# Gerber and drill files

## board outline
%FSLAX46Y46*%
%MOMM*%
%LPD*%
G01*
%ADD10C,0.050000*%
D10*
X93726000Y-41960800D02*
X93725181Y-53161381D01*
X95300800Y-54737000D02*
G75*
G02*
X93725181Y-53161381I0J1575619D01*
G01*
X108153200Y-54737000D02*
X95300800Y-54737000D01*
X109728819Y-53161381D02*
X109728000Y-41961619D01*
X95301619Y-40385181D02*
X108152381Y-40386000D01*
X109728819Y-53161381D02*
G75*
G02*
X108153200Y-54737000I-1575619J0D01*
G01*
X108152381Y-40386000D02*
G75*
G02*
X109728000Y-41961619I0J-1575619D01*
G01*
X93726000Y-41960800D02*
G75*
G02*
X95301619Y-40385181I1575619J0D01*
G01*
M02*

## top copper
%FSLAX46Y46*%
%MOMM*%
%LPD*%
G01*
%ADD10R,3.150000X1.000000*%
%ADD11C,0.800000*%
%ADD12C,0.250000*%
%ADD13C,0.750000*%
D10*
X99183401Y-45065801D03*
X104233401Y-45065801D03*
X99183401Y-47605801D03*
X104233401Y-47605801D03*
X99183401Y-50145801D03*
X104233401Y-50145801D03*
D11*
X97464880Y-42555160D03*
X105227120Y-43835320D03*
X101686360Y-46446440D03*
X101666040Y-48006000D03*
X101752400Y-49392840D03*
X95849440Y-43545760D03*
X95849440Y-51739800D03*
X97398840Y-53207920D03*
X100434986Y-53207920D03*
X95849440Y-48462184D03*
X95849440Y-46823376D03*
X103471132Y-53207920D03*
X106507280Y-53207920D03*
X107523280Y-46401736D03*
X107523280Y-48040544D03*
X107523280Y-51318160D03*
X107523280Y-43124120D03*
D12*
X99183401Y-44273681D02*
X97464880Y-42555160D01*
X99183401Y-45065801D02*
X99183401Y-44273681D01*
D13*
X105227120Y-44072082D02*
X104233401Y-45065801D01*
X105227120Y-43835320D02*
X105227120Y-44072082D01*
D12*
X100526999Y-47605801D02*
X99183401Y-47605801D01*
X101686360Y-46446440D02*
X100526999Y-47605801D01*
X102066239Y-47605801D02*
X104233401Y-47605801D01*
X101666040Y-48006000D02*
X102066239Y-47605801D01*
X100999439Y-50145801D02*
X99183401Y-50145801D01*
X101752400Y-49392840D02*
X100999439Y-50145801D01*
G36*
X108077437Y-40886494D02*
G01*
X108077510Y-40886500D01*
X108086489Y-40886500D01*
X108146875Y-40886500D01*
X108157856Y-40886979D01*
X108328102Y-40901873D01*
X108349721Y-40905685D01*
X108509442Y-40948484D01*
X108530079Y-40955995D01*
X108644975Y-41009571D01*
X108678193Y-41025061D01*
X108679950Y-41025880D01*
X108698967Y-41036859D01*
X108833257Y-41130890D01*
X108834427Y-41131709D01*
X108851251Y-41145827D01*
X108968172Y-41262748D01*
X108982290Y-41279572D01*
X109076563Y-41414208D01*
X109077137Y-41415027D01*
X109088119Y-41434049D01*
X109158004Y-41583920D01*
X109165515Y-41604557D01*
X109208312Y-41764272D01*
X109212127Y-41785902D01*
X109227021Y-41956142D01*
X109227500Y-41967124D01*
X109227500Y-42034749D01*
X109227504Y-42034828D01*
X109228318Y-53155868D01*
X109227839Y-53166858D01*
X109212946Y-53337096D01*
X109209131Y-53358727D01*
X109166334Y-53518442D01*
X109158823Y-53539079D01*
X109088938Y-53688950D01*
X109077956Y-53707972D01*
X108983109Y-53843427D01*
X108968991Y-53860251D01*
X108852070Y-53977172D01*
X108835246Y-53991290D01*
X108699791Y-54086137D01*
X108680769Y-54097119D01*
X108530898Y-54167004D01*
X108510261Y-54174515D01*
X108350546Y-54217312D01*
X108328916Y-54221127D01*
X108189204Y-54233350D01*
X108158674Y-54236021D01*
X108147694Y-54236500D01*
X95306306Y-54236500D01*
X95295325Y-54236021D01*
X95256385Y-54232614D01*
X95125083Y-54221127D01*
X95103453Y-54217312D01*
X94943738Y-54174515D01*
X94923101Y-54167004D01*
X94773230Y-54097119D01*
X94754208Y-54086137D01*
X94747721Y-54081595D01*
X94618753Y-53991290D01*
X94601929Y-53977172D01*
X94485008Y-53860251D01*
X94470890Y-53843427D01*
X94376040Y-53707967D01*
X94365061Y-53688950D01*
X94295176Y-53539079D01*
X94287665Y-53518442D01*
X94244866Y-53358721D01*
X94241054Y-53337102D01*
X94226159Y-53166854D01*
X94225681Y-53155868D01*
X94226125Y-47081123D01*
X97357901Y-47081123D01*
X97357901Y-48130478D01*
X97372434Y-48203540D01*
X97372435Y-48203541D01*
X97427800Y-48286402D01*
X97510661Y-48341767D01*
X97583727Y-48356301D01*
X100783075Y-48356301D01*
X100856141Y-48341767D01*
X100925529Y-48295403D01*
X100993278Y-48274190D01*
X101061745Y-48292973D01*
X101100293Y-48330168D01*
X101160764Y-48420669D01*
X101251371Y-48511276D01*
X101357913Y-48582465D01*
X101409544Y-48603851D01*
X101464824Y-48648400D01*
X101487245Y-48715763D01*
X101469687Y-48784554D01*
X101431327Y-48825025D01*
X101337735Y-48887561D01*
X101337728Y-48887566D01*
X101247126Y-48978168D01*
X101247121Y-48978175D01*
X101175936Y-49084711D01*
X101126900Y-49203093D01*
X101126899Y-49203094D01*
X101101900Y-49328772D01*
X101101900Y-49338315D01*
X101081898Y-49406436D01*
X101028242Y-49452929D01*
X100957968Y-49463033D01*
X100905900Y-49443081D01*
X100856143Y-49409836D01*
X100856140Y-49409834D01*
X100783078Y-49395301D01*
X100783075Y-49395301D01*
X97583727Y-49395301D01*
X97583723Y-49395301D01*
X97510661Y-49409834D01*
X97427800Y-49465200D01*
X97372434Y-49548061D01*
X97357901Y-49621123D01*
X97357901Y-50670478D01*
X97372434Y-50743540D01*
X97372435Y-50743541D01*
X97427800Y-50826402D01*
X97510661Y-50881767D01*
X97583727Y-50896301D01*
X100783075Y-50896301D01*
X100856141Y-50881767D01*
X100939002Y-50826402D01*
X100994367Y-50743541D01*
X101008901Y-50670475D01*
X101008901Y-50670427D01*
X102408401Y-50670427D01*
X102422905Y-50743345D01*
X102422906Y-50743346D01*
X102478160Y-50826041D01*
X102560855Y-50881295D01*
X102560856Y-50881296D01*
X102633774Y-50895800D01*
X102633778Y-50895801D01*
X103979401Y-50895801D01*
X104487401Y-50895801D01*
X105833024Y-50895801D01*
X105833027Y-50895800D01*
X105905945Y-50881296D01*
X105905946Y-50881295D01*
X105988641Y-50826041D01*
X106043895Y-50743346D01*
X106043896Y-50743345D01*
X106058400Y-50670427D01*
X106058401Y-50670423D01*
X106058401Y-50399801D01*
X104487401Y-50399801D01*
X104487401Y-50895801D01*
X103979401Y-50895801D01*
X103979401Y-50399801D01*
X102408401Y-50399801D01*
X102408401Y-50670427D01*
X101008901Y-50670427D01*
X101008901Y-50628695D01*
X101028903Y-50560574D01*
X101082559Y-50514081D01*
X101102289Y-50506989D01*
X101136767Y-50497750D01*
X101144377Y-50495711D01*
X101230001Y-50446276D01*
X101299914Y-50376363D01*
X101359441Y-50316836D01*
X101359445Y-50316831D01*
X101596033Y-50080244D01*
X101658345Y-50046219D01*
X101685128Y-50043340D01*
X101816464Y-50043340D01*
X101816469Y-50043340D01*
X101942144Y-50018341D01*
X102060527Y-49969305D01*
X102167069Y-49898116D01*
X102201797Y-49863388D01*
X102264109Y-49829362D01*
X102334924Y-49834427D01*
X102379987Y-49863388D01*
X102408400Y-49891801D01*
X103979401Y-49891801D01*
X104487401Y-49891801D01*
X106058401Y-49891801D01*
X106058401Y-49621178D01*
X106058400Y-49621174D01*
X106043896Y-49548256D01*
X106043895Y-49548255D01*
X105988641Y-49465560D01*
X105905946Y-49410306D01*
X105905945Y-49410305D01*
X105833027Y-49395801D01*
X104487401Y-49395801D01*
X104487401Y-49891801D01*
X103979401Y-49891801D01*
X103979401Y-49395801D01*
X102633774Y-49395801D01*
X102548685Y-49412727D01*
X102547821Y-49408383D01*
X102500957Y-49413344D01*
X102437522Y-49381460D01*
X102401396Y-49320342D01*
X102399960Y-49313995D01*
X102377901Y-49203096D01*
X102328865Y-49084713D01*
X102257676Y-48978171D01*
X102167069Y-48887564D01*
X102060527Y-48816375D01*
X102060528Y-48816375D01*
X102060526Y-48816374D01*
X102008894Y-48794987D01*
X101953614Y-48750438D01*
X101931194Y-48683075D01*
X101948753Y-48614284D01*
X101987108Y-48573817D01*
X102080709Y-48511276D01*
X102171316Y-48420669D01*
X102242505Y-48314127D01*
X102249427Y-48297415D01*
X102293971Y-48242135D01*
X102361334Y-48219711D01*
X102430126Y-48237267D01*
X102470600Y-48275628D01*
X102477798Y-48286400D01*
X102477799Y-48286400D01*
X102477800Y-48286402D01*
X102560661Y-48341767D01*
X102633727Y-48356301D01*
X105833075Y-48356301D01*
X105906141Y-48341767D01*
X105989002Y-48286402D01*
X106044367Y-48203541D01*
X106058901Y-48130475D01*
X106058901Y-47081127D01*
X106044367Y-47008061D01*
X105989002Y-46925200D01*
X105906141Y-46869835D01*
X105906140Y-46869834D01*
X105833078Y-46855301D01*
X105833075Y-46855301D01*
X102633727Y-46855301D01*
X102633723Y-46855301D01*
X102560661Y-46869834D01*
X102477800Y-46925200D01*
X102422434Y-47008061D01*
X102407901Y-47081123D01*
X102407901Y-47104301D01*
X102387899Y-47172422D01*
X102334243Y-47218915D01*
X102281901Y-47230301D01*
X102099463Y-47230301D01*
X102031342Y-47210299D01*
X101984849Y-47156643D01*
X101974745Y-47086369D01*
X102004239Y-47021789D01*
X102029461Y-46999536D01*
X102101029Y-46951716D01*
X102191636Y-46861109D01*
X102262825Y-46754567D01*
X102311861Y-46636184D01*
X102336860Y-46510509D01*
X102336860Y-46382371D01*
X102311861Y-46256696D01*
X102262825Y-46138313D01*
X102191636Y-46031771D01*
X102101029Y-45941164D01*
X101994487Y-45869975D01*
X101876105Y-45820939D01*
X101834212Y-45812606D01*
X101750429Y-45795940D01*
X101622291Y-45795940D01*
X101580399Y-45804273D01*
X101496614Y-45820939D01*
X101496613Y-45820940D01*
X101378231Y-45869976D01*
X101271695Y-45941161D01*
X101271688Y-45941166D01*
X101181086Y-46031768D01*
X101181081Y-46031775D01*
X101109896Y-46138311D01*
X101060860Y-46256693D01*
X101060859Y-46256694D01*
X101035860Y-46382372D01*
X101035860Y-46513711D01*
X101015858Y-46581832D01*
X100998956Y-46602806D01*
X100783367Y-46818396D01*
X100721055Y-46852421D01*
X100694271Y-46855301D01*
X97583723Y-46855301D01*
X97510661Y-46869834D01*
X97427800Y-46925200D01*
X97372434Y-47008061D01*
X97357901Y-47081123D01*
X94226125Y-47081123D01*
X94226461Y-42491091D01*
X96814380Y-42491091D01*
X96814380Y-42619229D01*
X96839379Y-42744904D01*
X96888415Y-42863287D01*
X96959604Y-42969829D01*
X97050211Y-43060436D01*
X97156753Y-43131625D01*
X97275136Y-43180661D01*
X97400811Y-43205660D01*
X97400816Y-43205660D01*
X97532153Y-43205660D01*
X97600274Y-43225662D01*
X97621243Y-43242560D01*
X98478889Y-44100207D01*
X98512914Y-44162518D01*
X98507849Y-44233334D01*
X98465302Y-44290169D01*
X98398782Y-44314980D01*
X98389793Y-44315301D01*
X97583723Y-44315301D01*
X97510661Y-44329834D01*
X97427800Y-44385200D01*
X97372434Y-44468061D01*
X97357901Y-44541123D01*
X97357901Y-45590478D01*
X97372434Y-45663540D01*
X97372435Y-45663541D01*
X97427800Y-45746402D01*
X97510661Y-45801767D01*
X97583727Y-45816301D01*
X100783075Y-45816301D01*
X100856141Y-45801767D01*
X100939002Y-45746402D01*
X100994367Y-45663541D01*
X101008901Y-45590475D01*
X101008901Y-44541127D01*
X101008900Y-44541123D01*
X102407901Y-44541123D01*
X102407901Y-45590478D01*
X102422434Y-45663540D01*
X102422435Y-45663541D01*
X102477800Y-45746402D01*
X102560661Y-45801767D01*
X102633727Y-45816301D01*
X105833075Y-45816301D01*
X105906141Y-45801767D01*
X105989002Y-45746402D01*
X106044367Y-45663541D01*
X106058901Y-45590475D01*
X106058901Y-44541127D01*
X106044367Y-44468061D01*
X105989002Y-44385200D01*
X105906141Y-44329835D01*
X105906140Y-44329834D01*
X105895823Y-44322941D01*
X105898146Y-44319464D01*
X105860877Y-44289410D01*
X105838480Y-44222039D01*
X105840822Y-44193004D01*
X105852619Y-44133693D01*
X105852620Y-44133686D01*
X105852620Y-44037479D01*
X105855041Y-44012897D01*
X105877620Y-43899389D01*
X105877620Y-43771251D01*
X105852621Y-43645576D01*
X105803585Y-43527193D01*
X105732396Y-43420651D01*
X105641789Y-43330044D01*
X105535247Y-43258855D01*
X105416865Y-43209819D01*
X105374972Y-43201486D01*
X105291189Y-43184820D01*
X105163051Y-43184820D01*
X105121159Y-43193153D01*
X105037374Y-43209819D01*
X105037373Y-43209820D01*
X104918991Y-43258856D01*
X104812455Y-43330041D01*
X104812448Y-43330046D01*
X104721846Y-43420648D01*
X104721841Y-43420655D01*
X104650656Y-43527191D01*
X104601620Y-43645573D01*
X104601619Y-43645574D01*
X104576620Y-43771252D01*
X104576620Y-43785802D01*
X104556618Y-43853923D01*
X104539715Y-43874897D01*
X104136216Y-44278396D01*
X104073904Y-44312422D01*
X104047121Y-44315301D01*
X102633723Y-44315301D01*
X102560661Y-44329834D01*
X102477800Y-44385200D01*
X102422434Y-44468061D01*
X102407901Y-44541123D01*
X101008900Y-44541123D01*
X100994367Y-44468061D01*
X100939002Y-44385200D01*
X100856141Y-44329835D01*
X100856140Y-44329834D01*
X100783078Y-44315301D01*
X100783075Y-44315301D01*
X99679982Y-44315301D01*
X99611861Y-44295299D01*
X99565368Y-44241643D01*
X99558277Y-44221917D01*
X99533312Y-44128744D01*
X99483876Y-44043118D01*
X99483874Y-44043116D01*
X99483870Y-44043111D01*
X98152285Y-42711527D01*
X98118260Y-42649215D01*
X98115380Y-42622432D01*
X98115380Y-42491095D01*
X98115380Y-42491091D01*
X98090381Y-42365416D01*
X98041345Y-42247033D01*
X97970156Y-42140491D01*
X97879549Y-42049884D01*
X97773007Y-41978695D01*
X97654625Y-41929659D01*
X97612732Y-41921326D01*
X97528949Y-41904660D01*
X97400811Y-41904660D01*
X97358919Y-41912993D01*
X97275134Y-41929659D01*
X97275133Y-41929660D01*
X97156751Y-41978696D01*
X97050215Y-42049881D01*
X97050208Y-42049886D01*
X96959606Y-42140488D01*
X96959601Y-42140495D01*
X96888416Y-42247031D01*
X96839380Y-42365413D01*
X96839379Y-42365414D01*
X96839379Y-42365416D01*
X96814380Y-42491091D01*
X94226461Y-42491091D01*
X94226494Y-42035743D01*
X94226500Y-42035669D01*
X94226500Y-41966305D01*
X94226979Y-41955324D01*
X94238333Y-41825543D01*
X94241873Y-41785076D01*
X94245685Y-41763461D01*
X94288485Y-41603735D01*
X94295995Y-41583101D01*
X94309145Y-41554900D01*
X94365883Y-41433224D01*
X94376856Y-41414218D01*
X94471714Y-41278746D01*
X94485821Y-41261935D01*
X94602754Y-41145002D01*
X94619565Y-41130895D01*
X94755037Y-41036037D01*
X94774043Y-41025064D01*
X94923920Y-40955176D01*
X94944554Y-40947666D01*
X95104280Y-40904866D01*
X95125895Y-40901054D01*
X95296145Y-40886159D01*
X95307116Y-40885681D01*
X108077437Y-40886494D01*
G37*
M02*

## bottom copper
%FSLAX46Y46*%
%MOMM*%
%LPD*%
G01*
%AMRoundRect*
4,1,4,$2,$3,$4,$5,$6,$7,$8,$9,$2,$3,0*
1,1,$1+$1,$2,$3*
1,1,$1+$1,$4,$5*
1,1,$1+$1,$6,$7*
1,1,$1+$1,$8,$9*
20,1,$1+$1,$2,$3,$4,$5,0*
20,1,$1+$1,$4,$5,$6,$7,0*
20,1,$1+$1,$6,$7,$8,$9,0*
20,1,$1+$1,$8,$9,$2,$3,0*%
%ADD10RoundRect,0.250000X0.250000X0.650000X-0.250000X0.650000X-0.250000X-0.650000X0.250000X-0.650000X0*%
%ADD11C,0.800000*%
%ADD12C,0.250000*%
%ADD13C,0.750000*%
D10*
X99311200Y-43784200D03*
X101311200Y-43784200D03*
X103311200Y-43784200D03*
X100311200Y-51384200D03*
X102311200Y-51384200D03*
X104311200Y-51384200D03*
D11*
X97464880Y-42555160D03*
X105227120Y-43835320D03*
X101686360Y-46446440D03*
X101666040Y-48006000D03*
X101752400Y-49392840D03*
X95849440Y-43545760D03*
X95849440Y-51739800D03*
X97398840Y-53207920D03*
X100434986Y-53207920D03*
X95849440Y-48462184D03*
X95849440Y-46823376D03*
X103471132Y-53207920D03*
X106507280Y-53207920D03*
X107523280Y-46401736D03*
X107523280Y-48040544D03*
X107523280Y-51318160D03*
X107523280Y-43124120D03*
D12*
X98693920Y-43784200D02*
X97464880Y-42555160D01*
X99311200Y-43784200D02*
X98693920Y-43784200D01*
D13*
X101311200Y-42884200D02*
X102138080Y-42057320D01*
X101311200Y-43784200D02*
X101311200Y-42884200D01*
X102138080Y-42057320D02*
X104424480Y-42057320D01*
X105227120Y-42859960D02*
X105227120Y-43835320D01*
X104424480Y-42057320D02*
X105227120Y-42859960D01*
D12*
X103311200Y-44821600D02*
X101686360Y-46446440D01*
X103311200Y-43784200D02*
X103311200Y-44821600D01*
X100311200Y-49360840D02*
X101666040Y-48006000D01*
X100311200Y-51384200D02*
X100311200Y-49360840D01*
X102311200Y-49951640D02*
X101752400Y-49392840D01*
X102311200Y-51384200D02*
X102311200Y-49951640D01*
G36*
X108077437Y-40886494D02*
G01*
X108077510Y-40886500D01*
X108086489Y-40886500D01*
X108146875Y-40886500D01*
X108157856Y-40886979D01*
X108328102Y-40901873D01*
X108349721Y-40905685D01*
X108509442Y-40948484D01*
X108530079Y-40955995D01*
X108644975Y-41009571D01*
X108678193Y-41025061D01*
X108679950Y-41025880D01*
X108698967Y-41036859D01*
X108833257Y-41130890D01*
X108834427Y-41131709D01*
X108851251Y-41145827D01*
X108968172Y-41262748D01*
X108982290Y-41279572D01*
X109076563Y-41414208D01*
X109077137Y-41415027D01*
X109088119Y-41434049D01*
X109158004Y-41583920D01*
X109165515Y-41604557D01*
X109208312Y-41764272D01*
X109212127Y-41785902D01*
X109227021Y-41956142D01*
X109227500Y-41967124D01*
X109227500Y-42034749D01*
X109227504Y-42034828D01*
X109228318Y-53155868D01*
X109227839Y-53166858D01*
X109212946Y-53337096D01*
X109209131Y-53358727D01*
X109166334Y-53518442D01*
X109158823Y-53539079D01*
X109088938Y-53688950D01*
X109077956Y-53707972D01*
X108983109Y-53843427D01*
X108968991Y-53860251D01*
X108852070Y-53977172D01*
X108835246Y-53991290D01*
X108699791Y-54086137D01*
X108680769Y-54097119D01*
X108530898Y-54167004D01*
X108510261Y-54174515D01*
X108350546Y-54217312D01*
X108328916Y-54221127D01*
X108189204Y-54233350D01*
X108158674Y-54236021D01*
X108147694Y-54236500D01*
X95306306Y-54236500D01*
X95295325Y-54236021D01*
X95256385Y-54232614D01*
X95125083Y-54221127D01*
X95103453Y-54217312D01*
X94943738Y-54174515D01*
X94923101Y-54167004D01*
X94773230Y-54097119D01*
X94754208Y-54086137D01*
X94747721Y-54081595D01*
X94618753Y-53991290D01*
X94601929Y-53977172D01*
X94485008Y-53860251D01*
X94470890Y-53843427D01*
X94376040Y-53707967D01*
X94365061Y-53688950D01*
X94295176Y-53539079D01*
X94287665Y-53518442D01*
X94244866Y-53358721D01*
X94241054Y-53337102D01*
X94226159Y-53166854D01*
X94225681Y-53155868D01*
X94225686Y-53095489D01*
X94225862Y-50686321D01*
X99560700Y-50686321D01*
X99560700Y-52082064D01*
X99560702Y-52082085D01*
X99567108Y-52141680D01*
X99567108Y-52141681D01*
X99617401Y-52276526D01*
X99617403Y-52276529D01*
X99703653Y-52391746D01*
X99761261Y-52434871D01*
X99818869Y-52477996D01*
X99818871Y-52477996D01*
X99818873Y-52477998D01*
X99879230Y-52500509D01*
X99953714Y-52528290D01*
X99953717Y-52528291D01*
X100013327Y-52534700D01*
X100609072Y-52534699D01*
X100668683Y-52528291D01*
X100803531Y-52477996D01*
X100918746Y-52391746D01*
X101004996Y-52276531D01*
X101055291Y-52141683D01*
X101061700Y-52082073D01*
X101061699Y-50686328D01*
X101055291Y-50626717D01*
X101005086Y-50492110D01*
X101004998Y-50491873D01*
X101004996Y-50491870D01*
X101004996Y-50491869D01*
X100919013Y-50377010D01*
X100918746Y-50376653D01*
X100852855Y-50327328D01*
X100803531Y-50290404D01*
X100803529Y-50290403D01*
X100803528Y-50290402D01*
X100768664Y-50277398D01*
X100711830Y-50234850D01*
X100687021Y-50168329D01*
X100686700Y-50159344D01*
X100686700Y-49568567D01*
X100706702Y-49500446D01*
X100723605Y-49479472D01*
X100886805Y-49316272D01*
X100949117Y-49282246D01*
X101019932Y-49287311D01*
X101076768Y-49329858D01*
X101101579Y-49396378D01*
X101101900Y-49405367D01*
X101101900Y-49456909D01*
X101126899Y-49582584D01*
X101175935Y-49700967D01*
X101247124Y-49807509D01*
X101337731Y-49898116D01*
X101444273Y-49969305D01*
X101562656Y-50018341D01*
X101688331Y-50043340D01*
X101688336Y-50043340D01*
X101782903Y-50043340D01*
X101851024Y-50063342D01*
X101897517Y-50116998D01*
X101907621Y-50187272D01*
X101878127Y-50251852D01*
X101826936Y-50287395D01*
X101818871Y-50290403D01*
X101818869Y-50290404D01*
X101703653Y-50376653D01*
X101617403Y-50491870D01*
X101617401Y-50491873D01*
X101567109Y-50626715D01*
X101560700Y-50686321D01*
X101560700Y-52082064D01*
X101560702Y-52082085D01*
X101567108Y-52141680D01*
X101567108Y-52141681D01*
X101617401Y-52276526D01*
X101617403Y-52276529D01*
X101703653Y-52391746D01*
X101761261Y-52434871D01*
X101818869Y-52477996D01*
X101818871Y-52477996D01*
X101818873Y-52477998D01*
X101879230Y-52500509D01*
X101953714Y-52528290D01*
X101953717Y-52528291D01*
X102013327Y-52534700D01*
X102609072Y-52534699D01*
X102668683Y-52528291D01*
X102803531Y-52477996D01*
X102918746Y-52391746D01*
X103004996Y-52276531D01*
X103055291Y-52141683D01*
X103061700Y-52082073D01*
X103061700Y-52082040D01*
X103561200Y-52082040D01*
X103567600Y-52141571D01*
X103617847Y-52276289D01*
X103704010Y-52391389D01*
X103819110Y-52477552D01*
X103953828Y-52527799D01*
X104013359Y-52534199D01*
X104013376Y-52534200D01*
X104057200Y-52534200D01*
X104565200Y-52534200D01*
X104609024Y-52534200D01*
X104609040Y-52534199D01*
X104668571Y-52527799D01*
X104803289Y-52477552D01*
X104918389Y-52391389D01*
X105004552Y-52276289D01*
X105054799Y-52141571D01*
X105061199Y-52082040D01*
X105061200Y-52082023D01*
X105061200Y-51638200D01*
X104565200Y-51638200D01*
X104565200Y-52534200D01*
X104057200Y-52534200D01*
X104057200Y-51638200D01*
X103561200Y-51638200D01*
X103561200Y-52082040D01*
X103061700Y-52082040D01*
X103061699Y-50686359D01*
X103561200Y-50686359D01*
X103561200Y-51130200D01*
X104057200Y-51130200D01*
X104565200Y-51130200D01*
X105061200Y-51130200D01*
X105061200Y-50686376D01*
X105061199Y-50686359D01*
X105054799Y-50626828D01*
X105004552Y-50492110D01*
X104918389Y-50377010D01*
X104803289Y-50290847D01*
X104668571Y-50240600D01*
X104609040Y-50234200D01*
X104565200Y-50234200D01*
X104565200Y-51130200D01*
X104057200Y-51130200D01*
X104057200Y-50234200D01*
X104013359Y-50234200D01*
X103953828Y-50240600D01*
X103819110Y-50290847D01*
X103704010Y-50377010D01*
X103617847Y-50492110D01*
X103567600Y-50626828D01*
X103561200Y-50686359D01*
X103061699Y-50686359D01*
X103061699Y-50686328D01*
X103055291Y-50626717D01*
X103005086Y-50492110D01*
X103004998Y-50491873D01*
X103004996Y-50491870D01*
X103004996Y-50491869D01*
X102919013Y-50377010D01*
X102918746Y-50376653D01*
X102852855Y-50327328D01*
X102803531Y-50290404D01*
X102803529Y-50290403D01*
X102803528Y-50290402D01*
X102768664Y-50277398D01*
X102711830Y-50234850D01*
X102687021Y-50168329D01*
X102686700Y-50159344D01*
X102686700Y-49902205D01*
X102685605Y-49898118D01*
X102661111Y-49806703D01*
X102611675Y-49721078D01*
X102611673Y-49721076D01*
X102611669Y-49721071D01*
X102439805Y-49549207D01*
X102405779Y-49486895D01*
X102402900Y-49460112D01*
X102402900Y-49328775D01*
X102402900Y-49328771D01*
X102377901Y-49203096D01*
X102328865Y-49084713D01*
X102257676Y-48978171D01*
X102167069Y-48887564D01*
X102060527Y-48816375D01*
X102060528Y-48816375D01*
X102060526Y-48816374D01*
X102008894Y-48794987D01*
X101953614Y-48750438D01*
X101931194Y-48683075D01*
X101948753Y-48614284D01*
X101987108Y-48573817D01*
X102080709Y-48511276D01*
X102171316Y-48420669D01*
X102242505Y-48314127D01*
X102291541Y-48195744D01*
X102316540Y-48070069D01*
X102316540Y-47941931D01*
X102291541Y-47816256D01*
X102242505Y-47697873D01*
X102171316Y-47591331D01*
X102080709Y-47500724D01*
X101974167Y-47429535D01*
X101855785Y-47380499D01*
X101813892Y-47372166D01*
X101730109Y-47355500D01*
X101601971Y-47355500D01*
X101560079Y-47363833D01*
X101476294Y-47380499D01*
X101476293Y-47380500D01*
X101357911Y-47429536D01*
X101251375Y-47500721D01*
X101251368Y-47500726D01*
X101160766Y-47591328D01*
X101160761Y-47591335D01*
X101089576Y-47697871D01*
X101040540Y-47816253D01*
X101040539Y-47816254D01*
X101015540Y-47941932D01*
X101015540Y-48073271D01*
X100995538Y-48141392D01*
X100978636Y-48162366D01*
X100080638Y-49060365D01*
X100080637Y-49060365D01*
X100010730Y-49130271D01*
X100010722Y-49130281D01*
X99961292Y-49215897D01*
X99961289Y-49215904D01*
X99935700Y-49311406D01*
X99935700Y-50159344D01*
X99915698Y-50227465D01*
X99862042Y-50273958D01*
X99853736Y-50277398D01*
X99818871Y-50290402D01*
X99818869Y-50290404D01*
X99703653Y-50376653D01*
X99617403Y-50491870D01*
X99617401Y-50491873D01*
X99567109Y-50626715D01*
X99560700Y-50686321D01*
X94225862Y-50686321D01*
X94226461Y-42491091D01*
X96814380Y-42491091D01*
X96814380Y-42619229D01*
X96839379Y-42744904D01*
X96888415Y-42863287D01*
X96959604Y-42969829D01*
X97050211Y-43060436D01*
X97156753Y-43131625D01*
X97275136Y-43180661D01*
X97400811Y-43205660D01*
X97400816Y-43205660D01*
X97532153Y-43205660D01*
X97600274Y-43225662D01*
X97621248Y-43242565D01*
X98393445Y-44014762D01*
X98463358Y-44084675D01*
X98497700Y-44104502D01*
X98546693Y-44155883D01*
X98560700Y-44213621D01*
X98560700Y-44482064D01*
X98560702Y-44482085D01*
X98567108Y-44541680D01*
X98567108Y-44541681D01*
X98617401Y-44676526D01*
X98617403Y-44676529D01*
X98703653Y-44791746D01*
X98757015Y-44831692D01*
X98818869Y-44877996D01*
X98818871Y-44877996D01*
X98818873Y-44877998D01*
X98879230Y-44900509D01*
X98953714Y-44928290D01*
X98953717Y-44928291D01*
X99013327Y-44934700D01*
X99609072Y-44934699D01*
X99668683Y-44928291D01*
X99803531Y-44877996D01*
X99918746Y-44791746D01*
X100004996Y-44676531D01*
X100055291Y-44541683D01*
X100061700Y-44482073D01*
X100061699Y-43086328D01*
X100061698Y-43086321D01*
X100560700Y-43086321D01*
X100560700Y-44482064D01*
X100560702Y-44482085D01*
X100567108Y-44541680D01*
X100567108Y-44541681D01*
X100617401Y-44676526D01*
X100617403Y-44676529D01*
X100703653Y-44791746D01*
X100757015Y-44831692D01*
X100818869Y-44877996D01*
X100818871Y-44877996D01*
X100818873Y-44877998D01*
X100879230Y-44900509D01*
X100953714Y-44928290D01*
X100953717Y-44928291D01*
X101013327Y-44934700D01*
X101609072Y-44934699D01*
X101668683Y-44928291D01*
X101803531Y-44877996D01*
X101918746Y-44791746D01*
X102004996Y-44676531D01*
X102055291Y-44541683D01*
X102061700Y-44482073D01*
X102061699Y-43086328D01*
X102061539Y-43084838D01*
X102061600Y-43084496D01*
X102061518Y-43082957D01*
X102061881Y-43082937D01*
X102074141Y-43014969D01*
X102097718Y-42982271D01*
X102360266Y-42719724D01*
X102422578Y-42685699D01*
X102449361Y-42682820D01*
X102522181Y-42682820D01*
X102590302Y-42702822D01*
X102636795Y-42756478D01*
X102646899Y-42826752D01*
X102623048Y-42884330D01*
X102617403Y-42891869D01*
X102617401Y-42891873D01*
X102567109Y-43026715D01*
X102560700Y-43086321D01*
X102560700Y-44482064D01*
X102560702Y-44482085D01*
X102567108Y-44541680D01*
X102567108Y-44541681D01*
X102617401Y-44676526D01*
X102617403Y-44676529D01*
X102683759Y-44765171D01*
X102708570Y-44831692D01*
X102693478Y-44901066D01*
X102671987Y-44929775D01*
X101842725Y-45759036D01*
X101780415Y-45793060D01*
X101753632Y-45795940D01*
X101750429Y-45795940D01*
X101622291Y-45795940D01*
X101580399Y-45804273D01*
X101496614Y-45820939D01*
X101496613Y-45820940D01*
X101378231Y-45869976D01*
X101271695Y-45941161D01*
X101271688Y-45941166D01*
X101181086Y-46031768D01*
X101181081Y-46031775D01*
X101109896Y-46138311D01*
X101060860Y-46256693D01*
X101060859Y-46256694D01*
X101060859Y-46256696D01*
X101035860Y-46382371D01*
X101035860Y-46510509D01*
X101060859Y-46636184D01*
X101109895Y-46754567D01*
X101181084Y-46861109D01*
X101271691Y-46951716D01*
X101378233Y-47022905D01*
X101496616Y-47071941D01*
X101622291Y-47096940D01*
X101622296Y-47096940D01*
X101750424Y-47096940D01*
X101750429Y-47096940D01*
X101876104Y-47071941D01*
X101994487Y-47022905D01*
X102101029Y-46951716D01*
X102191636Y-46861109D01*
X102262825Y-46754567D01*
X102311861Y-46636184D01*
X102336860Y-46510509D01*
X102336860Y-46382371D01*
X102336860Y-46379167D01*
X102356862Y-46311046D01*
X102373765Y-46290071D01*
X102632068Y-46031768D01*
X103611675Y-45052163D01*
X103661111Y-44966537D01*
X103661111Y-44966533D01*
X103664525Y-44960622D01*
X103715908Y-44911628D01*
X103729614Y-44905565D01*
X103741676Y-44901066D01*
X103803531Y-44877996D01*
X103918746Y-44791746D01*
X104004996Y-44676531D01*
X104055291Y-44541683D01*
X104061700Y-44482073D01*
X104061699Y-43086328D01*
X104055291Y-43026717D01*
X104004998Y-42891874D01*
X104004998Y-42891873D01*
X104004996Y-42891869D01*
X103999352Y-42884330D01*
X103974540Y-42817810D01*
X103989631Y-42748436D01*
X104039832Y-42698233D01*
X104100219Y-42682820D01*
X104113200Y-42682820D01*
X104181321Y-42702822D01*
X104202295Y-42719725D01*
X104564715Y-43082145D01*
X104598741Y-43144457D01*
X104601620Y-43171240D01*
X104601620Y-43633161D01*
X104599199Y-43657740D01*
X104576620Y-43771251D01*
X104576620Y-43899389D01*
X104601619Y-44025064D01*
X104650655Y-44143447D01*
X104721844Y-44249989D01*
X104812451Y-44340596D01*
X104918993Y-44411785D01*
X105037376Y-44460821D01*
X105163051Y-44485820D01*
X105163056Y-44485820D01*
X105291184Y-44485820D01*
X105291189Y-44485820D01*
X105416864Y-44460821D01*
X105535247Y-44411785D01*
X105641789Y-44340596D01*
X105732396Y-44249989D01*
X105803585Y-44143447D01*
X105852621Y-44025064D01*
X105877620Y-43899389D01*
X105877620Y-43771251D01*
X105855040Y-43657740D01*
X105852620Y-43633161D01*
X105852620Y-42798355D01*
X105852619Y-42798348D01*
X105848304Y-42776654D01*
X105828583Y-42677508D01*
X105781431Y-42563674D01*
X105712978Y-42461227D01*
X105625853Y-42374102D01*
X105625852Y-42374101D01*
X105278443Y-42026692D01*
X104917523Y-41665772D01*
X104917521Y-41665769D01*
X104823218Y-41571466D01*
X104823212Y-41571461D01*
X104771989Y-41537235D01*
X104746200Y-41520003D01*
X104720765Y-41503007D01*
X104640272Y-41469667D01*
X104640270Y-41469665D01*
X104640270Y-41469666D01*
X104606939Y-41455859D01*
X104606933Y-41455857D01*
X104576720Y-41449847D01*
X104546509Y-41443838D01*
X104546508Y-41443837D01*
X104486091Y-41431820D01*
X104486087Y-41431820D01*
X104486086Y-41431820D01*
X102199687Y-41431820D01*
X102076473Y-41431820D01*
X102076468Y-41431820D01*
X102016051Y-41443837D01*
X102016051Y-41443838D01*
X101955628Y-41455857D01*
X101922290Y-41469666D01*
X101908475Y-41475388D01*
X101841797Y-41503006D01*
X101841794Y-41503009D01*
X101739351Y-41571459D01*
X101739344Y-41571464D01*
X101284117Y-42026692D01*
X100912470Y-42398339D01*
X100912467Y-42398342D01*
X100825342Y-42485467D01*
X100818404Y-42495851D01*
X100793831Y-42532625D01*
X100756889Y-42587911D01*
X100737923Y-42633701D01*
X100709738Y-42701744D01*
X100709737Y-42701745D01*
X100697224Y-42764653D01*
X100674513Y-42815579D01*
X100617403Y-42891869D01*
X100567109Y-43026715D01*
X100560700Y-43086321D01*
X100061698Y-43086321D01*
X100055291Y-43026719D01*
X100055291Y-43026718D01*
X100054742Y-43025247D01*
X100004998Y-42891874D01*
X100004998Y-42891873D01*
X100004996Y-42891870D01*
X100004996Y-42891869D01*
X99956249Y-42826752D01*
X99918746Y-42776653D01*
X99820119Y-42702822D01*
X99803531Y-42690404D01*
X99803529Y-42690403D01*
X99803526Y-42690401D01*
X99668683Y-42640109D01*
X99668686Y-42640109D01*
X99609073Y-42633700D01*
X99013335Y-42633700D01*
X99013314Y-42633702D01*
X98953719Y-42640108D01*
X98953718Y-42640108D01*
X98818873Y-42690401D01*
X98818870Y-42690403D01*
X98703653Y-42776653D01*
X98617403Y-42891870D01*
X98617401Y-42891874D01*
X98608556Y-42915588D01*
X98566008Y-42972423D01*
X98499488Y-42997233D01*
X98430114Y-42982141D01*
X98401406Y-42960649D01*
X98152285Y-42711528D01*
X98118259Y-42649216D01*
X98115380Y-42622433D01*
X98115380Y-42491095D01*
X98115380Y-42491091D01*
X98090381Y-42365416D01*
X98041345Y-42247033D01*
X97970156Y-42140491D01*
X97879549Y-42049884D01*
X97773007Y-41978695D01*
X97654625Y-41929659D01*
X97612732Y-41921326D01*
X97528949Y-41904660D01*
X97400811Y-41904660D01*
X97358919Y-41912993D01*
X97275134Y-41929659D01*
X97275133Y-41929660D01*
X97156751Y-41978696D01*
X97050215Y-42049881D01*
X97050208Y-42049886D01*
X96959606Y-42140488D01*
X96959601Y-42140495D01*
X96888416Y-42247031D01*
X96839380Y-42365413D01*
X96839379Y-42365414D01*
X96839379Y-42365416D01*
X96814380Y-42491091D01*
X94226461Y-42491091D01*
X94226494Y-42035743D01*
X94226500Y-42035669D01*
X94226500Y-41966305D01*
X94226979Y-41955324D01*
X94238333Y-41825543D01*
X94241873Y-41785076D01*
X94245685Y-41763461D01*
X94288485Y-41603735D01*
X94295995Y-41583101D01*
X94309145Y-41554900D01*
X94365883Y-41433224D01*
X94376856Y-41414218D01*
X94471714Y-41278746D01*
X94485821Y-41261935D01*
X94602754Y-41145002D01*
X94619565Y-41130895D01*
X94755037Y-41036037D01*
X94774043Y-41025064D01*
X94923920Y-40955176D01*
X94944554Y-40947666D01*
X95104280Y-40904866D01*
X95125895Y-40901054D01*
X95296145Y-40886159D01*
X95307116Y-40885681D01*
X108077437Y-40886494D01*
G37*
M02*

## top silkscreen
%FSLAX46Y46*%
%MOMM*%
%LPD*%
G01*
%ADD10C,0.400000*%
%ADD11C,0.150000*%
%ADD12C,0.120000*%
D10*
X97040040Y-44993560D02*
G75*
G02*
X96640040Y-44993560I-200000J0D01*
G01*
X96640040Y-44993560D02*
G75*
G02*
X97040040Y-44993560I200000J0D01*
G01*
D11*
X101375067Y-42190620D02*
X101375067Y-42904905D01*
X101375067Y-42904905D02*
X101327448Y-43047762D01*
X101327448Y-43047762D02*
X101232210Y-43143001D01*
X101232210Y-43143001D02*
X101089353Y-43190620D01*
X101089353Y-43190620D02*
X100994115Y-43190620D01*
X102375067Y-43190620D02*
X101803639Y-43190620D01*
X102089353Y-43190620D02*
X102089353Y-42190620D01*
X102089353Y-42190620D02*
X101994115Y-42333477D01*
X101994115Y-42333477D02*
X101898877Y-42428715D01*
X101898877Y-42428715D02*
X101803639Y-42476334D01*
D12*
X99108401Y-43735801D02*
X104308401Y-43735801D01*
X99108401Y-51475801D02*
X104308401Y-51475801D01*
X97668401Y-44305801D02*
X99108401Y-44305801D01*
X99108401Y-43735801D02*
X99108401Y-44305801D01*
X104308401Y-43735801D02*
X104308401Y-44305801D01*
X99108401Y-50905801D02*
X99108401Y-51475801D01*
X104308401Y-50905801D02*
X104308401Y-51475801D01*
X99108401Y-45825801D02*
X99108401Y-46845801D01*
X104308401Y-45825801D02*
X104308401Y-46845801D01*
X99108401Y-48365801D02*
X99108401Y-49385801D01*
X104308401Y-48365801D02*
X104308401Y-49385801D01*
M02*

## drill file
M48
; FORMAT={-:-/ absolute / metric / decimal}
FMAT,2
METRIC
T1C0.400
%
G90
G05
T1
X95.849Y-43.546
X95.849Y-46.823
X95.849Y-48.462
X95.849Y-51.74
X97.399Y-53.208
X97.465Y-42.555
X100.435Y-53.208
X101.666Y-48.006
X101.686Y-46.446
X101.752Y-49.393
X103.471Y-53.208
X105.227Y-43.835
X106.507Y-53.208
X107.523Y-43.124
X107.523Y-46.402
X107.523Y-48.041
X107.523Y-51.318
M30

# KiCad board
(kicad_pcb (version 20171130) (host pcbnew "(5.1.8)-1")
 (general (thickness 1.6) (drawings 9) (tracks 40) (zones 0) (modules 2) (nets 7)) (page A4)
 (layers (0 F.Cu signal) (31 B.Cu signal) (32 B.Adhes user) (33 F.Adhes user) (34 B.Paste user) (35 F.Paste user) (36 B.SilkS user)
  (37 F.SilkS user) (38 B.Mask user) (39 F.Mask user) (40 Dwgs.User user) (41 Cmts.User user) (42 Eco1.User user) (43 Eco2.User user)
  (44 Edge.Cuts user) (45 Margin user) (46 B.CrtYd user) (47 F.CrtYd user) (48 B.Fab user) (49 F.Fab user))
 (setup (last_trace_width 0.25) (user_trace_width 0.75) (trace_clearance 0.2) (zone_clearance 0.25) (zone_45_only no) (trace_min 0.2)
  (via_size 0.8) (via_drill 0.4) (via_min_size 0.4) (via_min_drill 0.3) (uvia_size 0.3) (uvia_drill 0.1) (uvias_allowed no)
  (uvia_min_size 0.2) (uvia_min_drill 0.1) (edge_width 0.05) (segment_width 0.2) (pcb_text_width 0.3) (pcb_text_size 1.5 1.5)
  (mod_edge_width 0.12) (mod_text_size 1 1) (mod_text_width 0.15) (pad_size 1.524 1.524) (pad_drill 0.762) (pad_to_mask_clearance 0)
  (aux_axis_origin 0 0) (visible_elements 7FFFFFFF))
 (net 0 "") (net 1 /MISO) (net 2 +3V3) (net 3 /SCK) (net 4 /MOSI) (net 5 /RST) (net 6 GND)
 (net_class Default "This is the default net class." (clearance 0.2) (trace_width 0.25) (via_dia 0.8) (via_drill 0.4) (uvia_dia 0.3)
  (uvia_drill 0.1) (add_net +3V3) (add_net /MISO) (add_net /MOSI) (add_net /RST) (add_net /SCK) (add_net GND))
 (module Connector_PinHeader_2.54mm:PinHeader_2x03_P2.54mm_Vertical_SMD (layer F.Cu) (at 101.708401 47.605801)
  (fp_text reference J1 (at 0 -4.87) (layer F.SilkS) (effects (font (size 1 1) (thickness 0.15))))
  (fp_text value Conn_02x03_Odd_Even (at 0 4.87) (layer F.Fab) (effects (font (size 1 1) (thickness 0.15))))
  (fp_line (start -2.6 -3.87) (end 2.6 -3.87) (layer F.SilkS) (width 0.12))
  (fp_line (start -2.6 3.87) (end 2.6 3.87) (layer F.SilkS) (width 0.12))
  (fp_line (start -4.04 -3.3) (end -2.6 -3.3) (layer F.SilkS) (width 0.12))
  (fp_line (start -2.6 -3.87) (end -2.6 -3.3) (layer F.SilkS) (width 0.12))
  (fp_line (start 2.6 -3.87) (end 2.6 -3.3) (layer F.SilkS) (width 0.12))
  (fp_line (start -2.6 3.3) (end -2.6 3.87) (layer F.SilkS) (width 0.12))
  (fp_line (start 2.6 3.3) (end 2.6 3.87) (layer F.SilkS) (width 0.12))
  (fp_line (start -2.6 -1.78) (end -2.6 -0.76) (layer F.SilkS) (width 0.12))
  (fp_line (start 2.6 -1.78) (end 2.6 -0.76) (layer F.SilkS) (width 0.12))
  (fp_line (start -2.6 0.76) (end -2.6 1.78) (layer F.SilkS) (width 0.12))
  (fp_line (start 2.6 0.76) (end 2.6 1.78) (layer F.SilkS) (width 0.12))
  (pad 1 smd rect (at -2.525 -2.54) (size 3.15 1) (layers F.Cu F.Paste F.Mask) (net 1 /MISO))
  (pad 2 smd rect (at 2.525 -2.54) (size 3.15 1) (layers F.Cu F.Paste F.Mask) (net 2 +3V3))
  (pad 3 smd rect (at -2.525 0) (size 3.15 1) (layers F.Cu F.Paste F.Mask) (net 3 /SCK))
  (pad 4 smd rect (at 2.525 0) (size 3.15 1) (layers F.Cu F.Paste F.Mask) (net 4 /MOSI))
  (pad 5 smd rect (at -2.525 2.54) (size 3.15 1) (layers F.Cu F.Paste F.Mask) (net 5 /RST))
  (pad 6 smd rect (at 2.525 2.54) (size 3.15 1) (layers F.Cu F.Paste F.Mask) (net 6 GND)))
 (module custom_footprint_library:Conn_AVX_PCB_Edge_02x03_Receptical (layer B.Cu) (at 99.3112 43.7842)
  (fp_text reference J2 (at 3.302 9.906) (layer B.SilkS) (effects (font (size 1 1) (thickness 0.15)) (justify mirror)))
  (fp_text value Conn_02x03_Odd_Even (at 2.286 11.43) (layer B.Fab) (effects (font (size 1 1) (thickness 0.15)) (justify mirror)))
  (pad 1 smd roundrect (at 0 0 180) (size 1 1.8) (layers B.Cu B.Paste B.Mask) (roundrect_rratio 0.25) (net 1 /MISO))
  (pad 2 smd roundrect (at 2 0 180) (size 1 1.8) (layers B.Cu B.Paste B.Mask) (roundrect_rratio 0.25) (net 2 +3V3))
  (pad 3 smd roundrect (at 4 0 180) (size 1 1.8) (layers B.Cu B.Paste B.Mask) (roundrect_rratio 0.25) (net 3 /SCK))
  (pad 4 smd roundrect (at 1 7.6 180) (size 1 1.8) (layers B.Cu B.Paste B.Mask) (roundrect_rratio 0.25) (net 4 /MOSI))
  (pad 5 smd roundrect (at 3 7.6 180) (size 1 1.8) (layers B.Cu B.Paste B.Mask) (roundrect_rratio 0.25) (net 5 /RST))
  (pad 6 smd roundrect (at 5 7.6 180) (size 1 1.8) (layers B.Cu B.Paste B.Mask) (roundrect_rratio 0.25) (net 6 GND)))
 (gr_circle (center 96.84004 44.99356) (end 97.04004 44.99356) (layer F.SilkS) (width 0.4))
 (gr_line (start 93.726 41.9608) (end 93.725181 53.161381) (layer Edge.Cuts) (width 0.05))
 (gr_arc (start 95.3008 53.161381) (end 93.725181 53.161381) (angle -90) (layer Edge.Cuts) (width 0.05))
 (gr_line (start 108.1532 54.737) (end 95.3008 54.737) (layer Edge.Cuts) (width 0.05))
 (gr_line (start 109.728819 53.161381) (end 109.728 41.961619) (layer Edge.Cuts) (width 0.05))
 (gr_line (start 95.301619 40.385181) (end 108.152381 40.386) (layer Edge.Cuts) (width 0.05))
 (gr_arc (start 108.1532 53.161381) (end 108.1532 54.737) (angle -90) (layer Edge.Cuts) (width 0.05))
 (gr_arc (start 108.152381 41.961619) (end 109.728 41.961619) (angle -90) (layer Edge.Cuts) (width 0.05))
 (gr_arc (start 95.301619 41.9608) (end 95.301619 40.385181) (angle -90) (layer Edge.Cuts) (width 0.05))
 (via (at 97.46488 42.55516) (size 0.8) (drill 0.4) (layers F.Cu B.Cu) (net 1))
 (segment (start 99.183401 44.273681) (end 97.46488 42.55516) (width 0.25) (layer F.Cu) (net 1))
 (segment (start 99.183401 45.065801) (end 99.183401 44.273681) (width 0.25) (layer F.Cu) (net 1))
 (segment (start 98.69392 43.7842) (end 97.46488 42.55516) (width 0.25) (layer B.Cu) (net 1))
 (segment (start 99.3112 43.7842) (end 98.69392 43.7842) (width 0.25) (layer B.Cu) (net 1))
 (segment (start 101.3112 42.8842) (end 102.13808 42.05732) (width 0.75) (layer B.Cu) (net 2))
 (segment (start 101.3112 43.7842) (end 101.3112 42.8842) (width 0.75) (layer B.Cu) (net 2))
 (segment (start 102.13808 42.05732) (end 104.42448 42.05732) (width 0.75) (layer B.Cu) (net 2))
 (via (at 105.22712 43.83532) (size 0.8) (drill 0.4) (layers F.Cu B.Cu) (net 2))
 (segment (start 105.22712 42.85996) (end 105.22712 43.83532) (width 0.75) (layer B.Cu) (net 2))
 (segment (start 104.42448 42.05732) (end 105.22712 42.85996) (width 0.75) (layer B.Cu) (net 2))
 (segment (start 105.22712 44.072082) (end 104.233401 45.065801) (width 0.75) (layer F.Cu) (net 2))
 (segment (start 105.22712 43.83532) (end 105.22712 44.072082) (width 0.75) (layer F.Cu) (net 2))
 (via (at 101.68636 46.44644) (size 0.8) (drill 0.4) (layers F.Cu B.Cu) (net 3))
 (segment (start 103.3112 44.8216) (end 101.68636 46.44644) (width 0.25) (layer B.Cu) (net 3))
 (segment (start 103.3112 43.7842) (end 103.3112 44.8216) (width 0.25) (layer B.Cu) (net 3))
 (segment (start 100.526999 47.605801) (end 99.183401 47.605801) (width 0.25) (layer F.Cu) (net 3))
 (segment (start 101.68636 46.44644) (end 100.526999 47.605801) (width 0.25) (layer F.Cu) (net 3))
 (via (at 101.66604 48.006) (size 0.8) (drill 0.4) (layers F.Cu B.Cu) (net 4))
 (segment (start 100.3112 49.36084) (end 101.66604 48.006) (width 0.25) (layer B.Cu) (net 4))
 (segment (start 100.3112 51.3842) (end 100.3112 49.36084) (width 0.25) (layer B.Cu) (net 4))
 (segment (start 102.066239 47.605801) (end 104.233401 47.605801) (width 0.25) (layer F.Cu) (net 4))
 (segment (start 101.66604 48.006) (end 102.066239 47.605801) (width 0.25) (layer F.Cu) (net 4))
 (via (at 101.7524 49.39284) (size 0.8) (drill 0.4) (layers F.Cu B.Cu) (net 5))
 (segment (start 102.3112 49.95164) (end 101.7524 49.39284) (width 0.25) (layer B.Cu) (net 5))
 (segment (start 102.3112 51.3842) (end 102.3112 49.95164) (width 0.25) (layer B.Cu) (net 5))
 (segment (start 100.999439 50.145801) (end 99.183401 50.145801) (width 0.25) (layer F.Cu) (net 5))
 (segment (start 101.7524 49.39284) (end 100.999439 50.145801) (width 0.25) (layer F.Cu) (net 5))
 (via (at 95.84944 43.54576) (size 0.8) (drill 0.4) (layers F.Cu B.Cu) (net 6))
 (via (at 95.84944 51.7398) (size 0.8) (drill 0.4) (layers F.Cu B.Cu) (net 6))
 (via (at 97.39884 53.20792) (size 0.8) (drill 0.4) (layers F.Cu B.Cu) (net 6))
 (via (at 100.434986 53.20792) (size 0.8) (drill 0.4) (layers F.Cu B.Cu) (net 6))
 (via (at 95.84944 48.462184) (size 0.8) (drill 0.4) (layers F.Cu B.Cu) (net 6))
 (via (at 95.84944 46.823376) (size 0.8) (drill 0.4) (layers F.Cu B.Cu) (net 6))
 (via (at 103.471132 53.20792) (size 0.8) (drill 0.4) (layers F.Cu B.Cu) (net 6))
 (via (at 106.50728 53.20792) (size 0.8) (drill 0.4) (layers F.Cu B.Cu) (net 6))
 (via (at 107.52328 46.401736) (size 0.8) (drill 0.4) (layers F.Cu B.Cu) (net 6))
 (via (at 107.52328 48.040544) (size 0.8) (drill 0.4) (layers F.Cu B.Cu) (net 6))
 (via (at 107.52328 51.31816) (size 0.8) (drill 0.4) (layers F.Cu B.Cu) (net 6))
 (via (at 107.52328 43.12412) (size 0.8) (drill 0.4) (layers F.Cu B.Cu) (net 6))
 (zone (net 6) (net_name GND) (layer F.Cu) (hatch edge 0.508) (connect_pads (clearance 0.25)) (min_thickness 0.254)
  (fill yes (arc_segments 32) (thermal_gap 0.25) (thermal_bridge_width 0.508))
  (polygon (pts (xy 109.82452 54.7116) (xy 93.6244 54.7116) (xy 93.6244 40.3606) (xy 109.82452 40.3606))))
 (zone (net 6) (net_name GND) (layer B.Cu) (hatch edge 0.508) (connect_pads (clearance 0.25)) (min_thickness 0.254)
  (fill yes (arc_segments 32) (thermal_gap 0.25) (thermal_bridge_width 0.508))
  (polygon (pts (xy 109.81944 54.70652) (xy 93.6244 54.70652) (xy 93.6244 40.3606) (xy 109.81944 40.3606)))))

